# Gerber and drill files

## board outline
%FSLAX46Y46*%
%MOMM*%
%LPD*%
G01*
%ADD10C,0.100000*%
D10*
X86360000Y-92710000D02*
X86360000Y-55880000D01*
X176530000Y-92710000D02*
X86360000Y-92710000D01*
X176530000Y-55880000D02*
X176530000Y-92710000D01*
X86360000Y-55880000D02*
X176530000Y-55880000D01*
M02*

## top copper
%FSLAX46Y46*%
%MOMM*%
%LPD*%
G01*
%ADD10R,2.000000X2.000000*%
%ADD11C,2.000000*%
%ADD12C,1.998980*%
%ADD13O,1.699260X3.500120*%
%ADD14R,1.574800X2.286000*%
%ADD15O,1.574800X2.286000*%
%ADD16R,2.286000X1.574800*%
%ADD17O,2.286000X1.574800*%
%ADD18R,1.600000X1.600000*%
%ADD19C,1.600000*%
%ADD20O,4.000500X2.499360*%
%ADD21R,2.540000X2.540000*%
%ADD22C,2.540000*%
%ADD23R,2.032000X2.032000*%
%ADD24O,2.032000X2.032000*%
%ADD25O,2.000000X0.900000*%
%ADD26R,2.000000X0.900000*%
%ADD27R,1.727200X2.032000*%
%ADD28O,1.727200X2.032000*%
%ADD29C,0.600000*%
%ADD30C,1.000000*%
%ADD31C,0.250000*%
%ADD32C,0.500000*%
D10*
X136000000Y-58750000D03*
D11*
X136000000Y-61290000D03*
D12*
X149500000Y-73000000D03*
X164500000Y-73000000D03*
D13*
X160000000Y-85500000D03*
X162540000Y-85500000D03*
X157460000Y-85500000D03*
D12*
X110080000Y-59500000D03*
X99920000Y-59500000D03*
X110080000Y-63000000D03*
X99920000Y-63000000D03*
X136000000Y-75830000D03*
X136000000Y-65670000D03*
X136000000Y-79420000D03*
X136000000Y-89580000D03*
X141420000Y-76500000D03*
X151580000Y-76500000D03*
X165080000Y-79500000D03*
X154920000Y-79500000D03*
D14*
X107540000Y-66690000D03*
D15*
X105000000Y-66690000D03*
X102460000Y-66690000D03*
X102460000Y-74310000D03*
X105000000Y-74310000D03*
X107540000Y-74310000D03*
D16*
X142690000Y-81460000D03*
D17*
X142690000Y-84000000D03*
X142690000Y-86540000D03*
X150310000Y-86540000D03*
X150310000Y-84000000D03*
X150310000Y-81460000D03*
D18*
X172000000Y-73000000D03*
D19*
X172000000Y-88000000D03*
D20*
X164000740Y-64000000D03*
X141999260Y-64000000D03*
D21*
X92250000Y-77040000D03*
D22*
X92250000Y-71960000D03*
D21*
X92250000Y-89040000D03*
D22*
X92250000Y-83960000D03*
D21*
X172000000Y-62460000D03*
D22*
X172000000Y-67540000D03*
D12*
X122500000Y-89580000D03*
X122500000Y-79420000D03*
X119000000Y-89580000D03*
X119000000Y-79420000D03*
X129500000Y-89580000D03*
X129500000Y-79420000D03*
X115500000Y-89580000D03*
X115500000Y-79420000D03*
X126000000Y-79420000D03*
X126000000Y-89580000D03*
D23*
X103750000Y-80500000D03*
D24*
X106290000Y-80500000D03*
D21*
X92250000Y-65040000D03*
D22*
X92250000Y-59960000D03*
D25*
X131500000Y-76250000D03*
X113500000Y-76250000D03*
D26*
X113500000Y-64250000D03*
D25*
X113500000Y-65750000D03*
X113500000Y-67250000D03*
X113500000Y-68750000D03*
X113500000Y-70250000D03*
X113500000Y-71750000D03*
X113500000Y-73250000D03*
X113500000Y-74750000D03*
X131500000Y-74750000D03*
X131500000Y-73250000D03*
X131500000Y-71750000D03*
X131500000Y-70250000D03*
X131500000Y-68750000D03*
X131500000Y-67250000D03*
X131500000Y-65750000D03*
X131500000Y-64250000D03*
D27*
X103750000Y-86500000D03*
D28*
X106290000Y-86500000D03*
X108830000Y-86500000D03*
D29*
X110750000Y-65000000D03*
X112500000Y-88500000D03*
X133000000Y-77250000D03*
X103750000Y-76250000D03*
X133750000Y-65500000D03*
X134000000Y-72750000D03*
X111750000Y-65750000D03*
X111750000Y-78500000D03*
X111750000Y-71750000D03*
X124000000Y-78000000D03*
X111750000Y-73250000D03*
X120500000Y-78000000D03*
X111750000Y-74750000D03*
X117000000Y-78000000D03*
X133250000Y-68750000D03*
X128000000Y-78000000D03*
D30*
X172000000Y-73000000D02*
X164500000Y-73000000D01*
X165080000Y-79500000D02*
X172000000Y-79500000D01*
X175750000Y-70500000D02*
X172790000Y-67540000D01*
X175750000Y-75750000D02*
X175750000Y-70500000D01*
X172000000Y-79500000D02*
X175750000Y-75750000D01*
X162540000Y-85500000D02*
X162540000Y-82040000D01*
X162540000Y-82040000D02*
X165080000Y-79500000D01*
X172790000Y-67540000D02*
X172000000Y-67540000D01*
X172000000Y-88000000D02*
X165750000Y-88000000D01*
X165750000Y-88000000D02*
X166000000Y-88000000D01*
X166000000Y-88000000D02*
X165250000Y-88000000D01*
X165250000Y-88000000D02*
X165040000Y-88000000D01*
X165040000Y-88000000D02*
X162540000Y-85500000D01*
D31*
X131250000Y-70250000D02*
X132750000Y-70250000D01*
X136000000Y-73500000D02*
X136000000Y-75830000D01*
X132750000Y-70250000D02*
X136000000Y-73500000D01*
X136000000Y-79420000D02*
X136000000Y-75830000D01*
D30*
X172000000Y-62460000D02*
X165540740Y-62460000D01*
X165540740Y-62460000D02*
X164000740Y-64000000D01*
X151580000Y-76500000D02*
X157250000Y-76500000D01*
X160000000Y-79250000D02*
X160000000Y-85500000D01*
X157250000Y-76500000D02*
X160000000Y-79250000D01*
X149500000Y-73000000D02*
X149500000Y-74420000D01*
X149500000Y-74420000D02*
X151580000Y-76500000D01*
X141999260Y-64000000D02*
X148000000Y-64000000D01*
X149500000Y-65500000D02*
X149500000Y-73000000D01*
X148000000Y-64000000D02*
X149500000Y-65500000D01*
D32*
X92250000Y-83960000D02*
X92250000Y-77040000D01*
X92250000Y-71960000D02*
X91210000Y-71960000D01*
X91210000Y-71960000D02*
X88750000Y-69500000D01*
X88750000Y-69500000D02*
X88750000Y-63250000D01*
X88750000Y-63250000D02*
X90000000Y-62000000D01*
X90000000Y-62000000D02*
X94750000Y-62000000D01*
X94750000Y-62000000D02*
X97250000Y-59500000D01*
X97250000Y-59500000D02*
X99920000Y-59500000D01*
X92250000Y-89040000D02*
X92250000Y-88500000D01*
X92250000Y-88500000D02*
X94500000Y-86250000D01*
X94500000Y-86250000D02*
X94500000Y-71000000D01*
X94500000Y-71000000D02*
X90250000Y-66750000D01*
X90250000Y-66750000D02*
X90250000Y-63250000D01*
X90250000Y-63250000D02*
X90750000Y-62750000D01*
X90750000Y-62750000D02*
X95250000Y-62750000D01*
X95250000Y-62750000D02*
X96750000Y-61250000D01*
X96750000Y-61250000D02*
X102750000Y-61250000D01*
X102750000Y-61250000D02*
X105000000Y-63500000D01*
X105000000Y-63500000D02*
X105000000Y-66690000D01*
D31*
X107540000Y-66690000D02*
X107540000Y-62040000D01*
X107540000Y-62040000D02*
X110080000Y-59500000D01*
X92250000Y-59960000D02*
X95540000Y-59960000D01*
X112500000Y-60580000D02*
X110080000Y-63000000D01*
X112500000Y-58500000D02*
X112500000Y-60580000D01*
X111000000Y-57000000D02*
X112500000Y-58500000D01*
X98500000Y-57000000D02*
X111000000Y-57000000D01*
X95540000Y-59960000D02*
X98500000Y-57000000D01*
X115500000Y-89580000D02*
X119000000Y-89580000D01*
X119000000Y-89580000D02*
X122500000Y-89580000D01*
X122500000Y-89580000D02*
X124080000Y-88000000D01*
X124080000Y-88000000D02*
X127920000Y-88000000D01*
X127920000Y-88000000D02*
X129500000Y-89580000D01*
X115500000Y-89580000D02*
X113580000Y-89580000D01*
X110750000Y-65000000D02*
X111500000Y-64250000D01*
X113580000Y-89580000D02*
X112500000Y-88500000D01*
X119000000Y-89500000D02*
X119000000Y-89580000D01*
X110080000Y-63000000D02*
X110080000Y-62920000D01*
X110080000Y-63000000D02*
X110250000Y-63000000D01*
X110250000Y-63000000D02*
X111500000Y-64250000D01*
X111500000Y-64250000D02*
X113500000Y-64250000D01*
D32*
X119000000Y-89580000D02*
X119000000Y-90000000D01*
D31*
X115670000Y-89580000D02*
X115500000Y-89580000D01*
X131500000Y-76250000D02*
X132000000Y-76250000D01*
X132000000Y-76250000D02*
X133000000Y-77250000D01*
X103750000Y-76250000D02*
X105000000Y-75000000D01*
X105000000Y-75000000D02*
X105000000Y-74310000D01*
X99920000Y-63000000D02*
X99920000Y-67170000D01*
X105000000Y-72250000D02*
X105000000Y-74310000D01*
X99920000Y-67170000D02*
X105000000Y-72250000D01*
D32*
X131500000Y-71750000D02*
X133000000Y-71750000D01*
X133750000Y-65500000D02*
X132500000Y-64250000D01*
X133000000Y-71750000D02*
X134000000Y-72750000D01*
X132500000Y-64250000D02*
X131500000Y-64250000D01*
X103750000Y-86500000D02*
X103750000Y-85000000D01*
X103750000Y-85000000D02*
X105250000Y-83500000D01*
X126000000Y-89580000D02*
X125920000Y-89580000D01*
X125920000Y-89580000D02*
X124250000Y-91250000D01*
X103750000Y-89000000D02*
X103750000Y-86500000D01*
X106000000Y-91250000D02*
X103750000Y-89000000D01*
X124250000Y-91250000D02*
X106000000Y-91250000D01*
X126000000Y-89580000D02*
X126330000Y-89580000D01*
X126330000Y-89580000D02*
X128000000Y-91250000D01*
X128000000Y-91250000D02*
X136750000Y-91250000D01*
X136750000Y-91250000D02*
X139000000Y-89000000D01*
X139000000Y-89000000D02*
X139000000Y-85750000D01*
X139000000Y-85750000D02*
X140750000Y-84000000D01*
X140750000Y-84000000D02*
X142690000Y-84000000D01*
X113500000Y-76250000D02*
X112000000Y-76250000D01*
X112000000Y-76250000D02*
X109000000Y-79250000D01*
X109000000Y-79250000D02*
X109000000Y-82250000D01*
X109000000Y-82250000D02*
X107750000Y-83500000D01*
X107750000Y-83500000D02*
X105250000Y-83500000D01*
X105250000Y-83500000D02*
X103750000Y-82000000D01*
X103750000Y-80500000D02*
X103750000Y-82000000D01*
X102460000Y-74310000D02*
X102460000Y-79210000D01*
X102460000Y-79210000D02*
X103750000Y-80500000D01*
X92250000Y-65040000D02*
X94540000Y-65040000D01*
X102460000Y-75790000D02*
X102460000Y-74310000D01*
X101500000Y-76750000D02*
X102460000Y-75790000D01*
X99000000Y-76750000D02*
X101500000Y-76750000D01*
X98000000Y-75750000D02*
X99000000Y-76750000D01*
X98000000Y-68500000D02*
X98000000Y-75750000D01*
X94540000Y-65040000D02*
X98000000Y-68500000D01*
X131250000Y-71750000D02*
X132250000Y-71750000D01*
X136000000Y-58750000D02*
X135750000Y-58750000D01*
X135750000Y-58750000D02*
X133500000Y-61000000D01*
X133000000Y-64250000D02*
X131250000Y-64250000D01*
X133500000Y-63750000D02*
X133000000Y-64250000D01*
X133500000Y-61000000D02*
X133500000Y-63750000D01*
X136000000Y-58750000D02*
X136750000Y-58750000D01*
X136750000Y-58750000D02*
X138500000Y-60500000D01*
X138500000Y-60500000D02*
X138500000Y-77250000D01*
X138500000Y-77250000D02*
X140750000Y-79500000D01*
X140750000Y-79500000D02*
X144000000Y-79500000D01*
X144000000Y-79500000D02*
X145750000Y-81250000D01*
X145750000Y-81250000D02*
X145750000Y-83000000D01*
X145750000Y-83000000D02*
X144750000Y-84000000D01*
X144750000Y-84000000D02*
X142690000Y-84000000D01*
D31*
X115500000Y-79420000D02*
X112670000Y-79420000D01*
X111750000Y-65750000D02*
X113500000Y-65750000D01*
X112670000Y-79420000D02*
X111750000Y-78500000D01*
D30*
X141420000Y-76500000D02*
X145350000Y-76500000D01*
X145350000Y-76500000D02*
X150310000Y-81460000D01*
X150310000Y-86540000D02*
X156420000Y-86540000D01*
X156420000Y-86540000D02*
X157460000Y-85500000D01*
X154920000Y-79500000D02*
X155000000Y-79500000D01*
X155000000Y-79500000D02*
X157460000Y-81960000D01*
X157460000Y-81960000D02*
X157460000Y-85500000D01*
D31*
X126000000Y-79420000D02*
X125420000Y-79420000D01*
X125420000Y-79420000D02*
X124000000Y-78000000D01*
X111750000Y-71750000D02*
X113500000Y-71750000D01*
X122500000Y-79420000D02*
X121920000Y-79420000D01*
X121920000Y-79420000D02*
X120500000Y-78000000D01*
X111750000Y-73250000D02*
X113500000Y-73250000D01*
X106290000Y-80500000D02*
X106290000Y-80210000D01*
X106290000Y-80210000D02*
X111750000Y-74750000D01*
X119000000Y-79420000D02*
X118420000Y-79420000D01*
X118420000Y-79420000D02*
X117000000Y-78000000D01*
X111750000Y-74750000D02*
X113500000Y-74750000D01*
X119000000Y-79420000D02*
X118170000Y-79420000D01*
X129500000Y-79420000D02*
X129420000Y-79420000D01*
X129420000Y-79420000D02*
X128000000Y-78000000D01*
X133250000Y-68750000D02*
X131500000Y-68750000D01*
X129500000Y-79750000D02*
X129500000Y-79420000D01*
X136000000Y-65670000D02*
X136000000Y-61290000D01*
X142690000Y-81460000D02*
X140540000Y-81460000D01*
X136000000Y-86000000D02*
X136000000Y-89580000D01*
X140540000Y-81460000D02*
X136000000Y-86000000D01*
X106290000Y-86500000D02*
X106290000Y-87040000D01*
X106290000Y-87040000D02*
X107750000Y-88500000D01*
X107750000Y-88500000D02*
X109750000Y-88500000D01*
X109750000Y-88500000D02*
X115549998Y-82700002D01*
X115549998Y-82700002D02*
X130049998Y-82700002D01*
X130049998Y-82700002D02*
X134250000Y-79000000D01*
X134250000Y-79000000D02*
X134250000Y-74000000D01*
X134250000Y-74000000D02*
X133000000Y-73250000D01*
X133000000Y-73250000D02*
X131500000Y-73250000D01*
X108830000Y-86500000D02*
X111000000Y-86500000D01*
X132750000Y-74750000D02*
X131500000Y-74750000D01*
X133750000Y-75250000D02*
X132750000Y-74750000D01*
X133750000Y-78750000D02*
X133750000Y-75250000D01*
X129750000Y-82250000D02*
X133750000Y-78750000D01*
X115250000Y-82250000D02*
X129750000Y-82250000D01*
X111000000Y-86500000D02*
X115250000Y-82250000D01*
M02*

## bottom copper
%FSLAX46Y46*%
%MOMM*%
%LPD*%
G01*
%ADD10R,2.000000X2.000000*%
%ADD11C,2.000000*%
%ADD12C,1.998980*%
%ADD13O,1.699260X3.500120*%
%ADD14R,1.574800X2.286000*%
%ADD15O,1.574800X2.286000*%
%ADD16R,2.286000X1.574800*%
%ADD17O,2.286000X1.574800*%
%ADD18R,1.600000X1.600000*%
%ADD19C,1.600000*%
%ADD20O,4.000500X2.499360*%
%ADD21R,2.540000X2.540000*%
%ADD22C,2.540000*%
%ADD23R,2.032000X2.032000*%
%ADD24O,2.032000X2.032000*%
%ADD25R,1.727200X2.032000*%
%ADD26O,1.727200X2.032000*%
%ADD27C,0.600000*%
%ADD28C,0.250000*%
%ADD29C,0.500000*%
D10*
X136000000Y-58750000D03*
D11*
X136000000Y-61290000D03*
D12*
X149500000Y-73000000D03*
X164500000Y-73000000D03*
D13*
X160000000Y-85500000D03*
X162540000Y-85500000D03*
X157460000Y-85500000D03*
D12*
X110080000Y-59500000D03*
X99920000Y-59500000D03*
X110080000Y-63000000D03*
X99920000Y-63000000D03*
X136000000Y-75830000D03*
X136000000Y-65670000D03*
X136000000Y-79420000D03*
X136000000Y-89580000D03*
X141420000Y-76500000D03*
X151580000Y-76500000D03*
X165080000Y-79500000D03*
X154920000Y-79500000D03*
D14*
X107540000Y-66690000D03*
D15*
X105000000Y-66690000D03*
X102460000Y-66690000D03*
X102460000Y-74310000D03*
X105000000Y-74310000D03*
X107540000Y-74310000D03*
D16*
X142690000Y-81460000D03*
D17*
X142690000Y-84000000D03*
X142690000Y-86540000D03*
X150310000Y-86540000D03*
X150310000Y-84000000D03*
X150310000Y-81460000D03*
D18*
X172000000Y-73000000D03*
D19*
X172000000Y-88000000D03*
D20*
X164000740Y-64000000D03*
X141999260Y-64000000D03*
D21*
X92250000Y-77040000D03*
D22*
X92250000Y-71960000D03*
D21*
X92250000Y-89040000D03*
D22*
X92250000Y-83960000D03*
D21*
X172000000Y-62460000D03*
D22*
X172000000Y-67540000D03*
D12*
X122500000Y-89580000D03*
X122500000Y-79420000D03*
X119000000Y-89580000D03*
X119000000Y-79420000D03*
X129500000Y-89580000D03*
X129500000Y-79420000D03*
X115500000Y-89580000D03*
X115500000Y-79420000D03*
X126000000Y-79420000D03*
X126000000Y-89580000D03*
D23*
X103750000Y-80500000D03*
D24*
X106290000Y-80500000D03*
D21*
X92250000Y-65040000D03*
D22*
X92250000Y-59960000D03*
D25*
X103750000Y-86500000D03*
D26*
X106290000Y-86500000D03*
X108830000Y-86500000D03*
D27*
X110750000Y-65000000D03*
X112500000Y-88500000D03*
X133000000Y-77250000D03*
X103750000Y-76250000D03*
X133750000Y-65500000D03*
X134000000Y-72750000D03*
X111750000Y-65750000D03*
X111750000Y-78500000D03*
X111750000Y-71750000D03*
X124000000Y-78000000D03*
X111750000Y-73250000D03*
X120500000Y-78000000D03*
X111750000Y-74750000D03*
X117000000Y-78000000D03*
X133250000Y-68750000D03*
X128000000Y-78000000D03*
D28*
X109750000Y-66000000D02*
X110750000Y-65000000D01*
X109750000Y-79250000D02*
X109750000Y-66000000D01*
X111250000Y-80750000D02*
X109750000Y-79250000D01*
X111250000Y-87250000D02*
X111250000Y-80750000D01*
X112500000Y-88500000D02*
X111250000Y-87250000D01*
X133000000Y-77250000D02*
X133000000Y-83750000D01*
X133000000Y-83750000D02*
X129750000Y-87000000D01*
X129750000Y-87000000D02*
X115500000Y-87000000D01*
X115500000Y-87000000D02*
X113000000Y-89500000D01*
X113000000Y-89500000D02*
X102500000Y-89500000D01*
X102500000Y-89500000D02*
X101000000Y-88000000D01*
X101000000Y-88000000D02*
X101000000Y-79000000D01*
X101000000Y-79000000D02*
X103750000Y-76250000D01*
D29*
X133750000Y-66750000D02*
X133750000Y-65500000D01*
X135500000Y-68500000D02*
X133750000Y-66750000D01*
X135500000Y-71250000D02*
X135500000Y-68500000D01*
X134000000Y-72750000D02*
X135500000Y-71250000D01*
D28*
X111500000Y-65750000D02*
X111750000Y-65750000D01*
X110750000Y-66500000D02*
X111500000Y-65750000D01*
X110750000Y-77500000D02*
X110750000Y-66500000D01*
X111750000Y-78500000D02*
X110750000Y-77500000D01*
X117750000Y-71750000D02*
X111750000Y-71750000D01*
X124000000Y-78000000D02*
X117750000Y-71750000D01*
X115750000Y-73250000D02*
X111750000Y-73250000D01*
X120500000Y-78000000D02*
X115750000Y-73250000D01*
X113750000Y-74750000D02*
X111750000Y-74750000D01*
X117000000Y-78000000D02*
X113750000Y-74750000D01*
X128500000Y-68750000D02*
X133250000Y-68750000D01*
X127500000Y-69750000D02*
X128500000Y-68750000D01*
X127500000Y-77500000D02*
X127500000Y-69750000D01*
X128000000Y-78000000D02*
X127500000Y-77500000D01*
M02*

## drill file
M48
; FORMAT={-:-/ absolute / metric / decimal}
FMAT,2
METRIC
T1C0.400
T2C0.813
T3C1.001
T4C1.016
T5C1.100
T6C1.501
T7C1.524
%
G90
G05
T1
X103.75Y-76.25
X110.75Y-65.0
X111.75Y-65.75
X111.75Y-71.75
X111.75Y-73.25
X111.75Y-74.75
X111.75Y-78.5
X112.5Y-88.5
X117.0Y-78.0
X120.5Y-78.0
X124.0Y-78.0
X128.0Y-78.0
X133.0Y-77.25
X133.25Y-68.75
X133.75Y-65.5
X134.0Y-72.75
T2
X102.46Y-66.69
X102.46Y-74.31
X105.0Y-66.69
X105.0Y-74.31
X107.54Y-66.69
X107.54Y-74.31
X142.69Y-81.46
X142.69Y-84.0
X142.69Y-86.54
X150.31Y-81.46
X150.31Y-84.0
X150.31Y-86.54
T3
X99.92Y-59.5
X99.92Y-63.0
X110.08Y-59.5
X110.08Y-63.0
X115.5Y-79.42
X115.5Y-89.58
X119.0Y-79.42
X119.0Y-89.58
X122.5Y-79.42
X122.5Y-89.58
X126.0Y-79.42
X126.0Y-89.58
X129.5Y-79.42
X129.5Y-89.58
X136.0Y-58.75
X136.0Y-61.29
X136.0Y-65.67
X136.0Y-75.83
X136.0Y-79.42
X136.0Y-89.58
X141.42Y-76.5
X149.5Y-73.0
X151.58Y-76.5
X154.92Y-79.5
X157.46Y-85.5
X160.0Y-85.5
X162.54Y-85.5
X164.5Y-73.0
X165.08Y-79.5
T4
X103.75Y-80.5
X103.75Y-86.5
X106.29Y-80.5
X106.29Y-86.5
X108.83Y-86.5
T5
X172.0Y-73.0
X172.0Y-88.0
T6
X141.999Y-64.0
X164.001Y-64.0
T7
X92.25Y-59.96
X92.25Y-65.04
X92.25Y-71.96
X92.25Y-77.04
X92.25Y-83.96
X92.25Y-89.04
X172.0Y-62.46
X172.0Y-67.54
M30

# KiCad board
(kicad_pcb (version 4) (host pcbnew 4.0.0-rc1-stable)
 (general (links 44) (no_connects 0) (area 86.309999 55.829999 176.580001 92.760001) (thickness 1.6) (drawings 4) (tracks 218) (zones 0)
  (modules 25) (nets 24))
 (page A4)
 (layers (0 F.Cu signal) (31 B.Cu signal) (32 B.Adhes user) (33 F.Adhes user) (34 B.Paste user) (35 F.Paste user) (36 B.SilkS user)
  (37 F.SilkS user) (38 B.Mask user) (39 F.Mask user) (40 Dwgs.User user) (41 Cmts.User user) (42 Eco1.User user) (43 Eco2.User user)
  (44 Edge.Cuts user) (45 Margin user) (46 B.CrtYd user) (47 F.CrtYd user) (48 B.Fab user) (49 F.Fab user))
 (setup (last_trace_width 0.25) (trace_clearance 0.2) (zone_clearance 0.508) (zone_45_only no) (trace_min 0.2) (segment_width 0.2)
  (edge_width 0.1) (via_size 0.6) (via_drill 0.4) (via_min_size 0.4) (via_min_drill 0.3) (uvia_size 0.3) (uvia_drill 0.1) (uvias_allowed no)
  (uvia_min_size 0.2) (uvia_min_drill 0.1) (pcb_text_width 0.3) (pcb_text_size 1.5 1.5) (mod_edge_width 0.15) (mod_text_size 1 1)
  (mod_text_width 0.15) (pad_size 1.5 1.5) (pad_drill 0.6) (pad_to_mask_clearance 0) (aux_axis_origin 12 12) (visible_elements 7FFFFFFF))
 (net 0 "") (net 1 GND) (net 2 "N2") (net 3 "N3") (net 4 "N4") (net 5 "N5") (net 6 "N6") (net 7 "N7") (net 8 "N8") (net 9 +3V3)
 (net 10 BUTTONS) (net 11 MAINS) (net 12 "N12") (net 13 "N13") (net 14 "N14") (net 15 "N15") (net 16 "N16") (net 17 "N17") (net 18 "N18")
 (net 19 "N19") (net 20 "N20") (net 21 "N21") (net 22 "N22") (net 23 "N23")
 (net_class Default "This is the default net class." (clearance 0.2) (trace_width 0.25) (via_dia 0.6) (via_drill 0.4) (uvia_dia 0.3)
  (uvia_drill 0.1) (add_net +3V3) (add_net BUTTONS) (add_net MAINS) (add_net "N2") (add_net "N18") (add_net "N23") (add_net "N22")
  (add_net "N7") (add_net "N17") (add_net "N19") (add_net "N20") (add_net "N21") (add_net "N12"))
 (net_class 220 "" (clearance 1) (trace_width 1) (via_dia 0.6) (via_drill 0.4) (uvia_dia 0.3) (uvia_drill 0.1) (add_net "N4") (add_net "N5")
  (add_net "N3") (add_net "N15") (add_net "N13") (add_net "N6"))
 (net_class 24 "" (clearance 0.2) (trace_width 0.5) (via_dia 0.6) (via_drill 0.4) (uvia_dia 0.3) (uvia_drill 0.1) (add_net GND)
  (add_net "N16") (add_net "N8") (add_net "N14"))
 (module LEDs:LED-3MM (layer F.Cu) (at 136 58.75 270)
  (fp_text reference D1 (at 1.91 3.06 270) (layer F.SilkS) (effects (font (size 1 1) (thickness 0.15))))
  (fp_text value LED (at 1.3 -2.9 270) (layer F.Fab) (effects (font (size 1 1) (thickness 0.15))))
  (pad 1 thru_hole rect (at 0 0) (size 2 2) (drill 1.00076) (layers *.Cu *.Mask F.SilkS) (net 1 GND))
  (pad 2 thru_hole circle (at 2.54 0 270) (size 2 2) (drill 1.00076) (layers *.Cu *.Mask F.SilkS) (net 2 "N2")))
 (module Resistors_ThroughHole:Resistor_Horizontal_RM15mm (layer F.Cu) (at 157 73)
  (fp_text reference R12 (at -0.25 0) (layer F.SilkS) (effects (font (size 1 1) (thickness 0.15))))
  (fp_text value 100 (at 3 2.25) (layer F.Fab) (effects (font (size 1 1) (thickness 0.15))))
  (pad 1 thru_hole circle (at -7.5 0) (size 1.99898 1.99898) (drill 1.00076) (layers *.Cu *.SilkS *.Mask) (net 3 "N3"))
  (pad 2 thru_hole circle (at 7.5 0) (size 1.99898 1.99898) (drill 1.00076) (layers *.Cu *.SilkS *.Mask) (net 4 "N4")))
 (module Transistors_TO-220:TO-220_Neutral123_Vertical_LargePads (layer F.Cu) (at 160 85.5 180)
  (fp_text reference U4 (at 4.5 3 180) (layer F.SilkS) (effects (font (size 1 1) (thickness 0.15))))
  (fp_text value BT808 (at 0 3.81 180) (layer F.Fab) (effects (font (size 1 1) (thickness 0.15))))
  (pad 2 thru_hole oval (at 0 0 270) (size 3.50012 1.69926) (drill 1.00076) (layers *.Cu *.Mask F.SilkS) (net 3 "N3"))
  (pad 1 thru_hole oval (at -2.54 0 270) (size 3.50012 1.69926) (drill 1.00076) (layers *.Cu *.Mask F.SilkS) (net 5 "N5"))
  (pad 3 thru_hole oval (at 2.54 0 270) (size 3.50012 1.69926) (drill 1.00076) (layers *.Cu *.Mask F.SilkS) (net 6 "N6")))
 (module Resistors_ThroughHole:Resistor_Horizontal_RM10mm (layer F.Cu) (at 105 59.5 180)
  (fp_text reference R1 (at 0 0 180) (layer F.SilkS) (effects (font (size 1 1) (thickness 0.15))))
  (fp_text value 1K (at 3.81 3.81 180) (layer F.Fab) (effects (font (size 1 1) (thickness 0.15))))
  (pad 1 thru_hole circle (at -5.08 0 180) (size 1.99898 1.99898) (drill 1.00076) (layers *.Cu *.SilkS *.Mask) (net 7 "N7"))
  (pad 2 thru_hole circle (at 5.08 0 180) (size 1.99898 1.99898) (drill 1.00076) (layers *.Cu *.SilkS *.Mask) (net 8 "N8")))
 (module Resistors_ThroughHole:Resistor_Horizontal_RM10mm (layer F.Cu) (at 105 63 180)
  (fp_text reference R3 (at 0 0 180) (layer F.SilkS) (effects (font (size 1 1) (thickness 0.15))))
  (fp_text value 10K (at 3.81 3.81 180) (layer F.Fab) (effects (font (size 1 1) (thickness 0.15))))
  (pad 1 thru_hole circle (at -5.08 0 180) (size 1.99898 1.99898) (drill 1.00076) (layers *.Cu *.SilkS *.Mask) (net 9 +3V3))
  (pad 2 thru_hole circle (at 5.08 0 180) (size 1.99898 1.99898) (drill 1.00076) (layers *.Cu *.SilkS *.Mask) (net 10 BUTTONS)))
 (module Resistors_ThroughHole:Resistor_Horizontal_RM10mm (layer F.Cu) (at 136 70.75 90)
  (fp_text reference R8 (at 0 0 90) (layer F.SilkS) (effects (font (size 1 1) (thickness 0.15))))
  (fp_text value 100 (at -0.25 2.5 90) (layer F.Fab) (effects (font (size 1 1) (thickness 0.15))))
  (pad 1 thru_hole circle (at -5.08 0 90) (size 1.99898 1.99898) (drill 1.00076) (layers *.Cu *.SilkS *.Mask) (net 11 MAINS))
  (pad 2 thru_hole circle (at 5.08 0 90) (size 1.99898 1.99898) (drill 1.00076) (layers *.Cu *.SilkS *.Mask) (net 2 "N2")))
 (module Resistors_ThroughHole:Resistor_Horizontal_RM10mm (layer F.Cu) (at 136 84.5 270)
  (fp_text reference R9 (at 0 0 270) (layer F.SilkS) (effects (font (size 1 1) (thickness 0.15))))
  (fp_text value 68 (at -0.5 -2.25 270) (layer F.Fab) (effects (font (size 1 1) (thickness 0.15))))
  (pad 1 thru_hole circle (at -5.08 0 270) (size 1.99898 1.99898) (drill 1.00076) (layers *.Cu *.SilkS *.Mask) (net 11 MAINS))
  (pad 2 thru_hole circle (at 5.08 0 270) (size 1.99898 1.99898) (drill 1.00076) (layers *.Cu *.SilkS *.Mask) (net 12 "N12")))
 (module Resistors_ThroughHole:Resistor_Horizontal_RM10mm (layer F.Cu) (at 146.5 76.5)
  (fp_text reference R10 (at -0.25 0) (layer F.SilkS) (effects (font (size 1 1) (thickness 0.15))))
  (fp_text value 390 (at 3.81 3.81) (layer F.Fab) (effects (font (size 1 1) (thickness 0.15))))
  (pad 1 thru_hole circle (at -5.08 0) (size 1.99898 1.99898) (drill 1.00076) (layers *.Cu *.SilkS *.Mask) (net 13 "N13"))
  (pad 2 thru_hole circle (at 5.08 0) (size 1.99898 1.99898) (drill 1.00076) (layers *.Cu *.SilkS *.Mask) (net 3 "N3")))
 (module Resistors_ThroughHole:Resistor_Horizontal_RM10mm (layer F.Cu) (at 160 79.5 180)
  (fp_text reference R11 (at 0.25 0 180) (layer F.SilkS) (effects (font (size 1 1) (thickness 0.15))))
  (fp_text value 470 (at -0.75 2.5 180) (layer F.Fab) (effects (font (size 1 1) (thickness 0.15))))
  (pad 1 thru_hole circle (at -5.08 0 180) (size 1.99898 1.99898) (drill 1.00076) (layers *.Cu *.SilkS *.Mask) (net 5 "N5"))
  (pad 2 thru_hole circle (at 5.08 0 180) (size 1.99898 1.99898) (drill 1.00076) (layers *.Cu *.SilkS *.Mask) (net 6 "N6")))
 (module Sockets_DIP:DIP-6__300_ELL (layer F.Cu) (at 105 70.5 180)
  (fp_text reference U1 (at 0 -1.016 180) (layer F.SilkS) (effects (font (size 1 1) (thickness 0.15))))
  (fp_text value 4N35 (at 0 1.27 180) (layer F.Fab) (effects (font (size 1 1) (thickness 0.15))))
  (pad 1 thru_hole rect (at -2.54 3.81 180) (size 1.5748 2.286) (drill 0.8128) (layers *.Cu *.Mask F.SilkS) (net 7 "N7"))
  (pad 2 thru_hole oval (at 0 3.81 180) (size 1.5748 2.286) (drill 0.8128) (layers *.Cu *.Mask F.SilkS) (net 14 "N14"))
  (pad 3 thru_hole oval (at 2.54 3.81 180) (size 1.5748 2.286) (drill 0.8128) (layers *.Cu *.Mask F.SilkS))
  (pad 4 thru_hole oval (at 2.54 -3.81 180) (size 1.5748 2.286) (drill 0.8128) (layers *.Cu *.Mask F.SilkS) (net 1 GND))
  (pad 5 thru_hole oval (at 0 -3.81 180) (size 1.5748 2.286) (drill 0.8128) (layers *.Cu *.Mask F.SilkS) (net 10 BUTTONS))
  (pad 6 thru_hole oval (at -2.54 -3.81 180) (size 1.5748 2.286) (drill 0.8128) (layers *.Cu *.Mask F.SilkS)))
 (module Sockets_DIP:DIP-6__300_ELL (layer F.Cu) (at 146.5 84 270)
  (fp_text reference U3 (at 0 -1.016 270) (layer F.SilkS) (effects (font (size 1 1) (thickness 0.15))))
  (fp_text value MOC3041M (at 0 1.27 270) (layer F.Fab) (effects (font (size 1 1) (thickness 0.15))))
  (pad 1 thru_hole rect (at -2.54 3.81 270) (size 1.5748 2.286) (drill 0.8128) (layers *.Cu *.Mask F.SilkS) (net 12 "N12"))
  (pad 2 thru_hole oval (at 0 3.81 270) (size 1.5748 2.286) (drill 0.8128) (layers *.Cu *.Mask F.SilkS) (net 1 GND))
  (pad 3 thru_hole oval (at 2.54 3.81 270) (size 1.5748 2.286) (drill 0.8128) (layers *.Cu *.Mask F.SilkS))
  (pad 4 thru_hole oval (at 2.54 -3.81 270) (size 1.5748 2.286) (drill 0.8128) (layers *.Cu *.Mask F.SilkS) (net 6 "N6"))
  (pad 5 thru_hole oval (at 0 -3.81 270) (size 1.5748 2.286) (drill 0.8128) (layers *.Cu *.Mask F.SilkS))
  (pad 6 thru_hole oval (at -2.54 -3.81 270) (size 1.5748 2.286) (drill 0.8128) (layers *.Cu *.Mask F.SilkS) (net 13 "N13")))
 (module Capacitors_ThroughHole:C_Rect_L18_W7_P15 (layer F.Cu) (at 172 73 270)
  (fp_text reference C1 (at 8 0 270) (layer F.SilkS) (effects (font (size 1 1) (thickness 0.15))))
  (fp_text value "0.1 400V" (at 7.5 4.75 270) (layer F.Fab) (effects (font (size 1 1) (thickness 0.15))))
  (pad 1 thru_hole rect (at 0 0 270) (size 1.6 1.6) (drill 1.1) (layers *.Cu *.Mask F.SilkS) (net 4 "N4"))
  (pad 2 thru_hole circle (at 15 0 270) (size 1.6 1.6) (drill 1.1) (layers *.Cu *.Mask F.SilkS) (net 5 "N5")))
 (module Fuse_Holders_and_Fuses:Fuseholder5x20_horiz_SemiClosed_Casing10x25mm (layer F.Cu) (at 153 64)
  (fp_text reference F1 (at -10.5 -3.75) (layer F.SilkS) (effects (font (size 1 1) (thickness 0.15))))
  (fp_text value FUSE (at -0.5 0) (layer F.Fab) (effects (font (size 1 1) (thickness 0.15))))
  (pad 2 thru_hole oval (at 11.00074 0 270) (size 2.49936 4.0005) (drill 1.50114) (layers *.Cu *.Mask F.SilkS) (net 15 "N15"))
  (pad 1 thru_hole oval (at -11.00074 0 270) (size 2.49936 4.0005) (drill 1.50114) (layers *.Cu *.Mask F.SilkS) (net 3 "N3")))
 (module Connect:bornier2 (layer F.Cu) (at 92.25 74.5 90)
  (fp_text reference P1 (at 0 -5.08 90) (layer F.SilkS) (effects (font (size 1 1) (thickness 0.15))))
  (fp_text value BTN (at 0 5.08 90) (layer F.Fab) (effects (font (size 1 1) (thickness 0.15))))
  (pad 1 thru_hole rect (at -2.54 0 90) (size 2.54 2.54) (drill 1.524) (layers *.Cu *.Mask F.SilkS) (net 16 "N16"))
  (pad 2 thru_hole circle (at 2.54 0 90) (size 2.54 2.54) (drill 1.524) (layers *.Cu *.Mask F.SilkS) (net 8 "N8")))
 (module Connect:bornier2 (layer F.Cu) (at 92.25 86.5 90)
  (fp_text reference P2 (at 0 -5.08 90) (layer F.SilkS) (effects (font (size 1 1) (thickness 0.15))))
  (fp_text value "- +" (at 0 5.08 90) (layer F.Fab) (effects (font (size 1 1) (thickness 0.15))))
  (pad 1 thru_hole rect (at -2.54 0 90) (size 2.54 2.54) (drill 1.524) (layers *.Cu *.Mask F.SilkS) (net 14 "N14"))
  (pad 2 thru_hole circle (at 2.54 0 90) (size 2.54 2.54) (drill 1.524) (layers *.Cu *.Mask F.SilkS) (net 16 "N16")))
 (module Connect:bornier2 (layer F.Cu) (at 172 65 270)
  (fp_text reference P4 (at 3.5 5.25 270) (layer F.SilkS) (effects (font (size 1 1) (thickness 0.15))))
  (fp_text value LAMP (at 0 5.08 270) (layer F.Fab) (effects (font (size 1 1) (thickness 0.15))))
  (pad 1 thru_hole rect (at -2.54 0 270) (size 2.54 2.54) (drill 1.524) (layers *.Cu *.Mask F.SilkS) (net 15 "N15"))
  (pad 2 thru_hole circle (at 2.54 0 270) (size 2.54 2.54) (drill 1.524) (layers *.Cu *.Mask F.SilkS) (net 5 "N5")))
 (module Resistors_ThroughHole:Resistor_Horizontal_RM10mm (layer F.Cu) (at 122.5 84.5 90)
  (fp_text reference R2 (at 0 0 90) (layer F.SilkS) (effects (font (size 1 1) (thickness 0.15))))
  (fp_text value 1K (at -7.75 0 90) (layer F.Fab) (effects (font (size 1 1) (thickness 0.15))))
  (pad 1 thru_hole circle (at -5.08 0 90) (size 1.99898 1.99898) (drill 1.00076) (layers *.Cu *.SilkS *.Mask) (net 9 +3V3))
  (pad 2 thru_hole circle (at 5.08 0 90) (size 1.99898 1.99898) (drill 1.00076) (layers *.Cu *.SilkS *.Mask) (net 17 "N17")))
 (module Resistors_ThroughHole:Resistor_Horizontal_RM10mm (layer F.Cu) (at 119 84.5 90)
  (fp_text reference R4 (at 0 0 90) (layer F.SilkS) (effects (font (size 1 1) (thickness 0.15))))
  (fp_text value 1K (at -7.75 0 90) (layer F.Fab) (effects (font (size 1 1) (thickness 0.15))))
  (pad 1 thru_hole circle (at -5.08 0 90) (size 1.99898 1.99898) (drill 1.00076) (layers *.Cu *.SilkS *.Mask) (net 9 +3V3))
  (pad 2 thru_hole circle (at 5.08 0 90) (size 1.99898 1.99898) (drill 1.00076) (layers *.Cu *.SilkS *.Mask) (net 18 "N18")))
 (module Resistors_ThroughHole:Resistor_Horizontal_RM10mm (layer F.Cu) (at 129.5 84.5 90)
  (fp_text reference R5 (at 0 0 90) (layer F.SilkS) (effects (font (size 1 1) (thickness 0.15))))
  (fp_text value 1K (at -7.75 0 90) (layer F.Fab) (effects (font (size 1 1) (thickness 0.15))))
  (pad 1 thru_hole circle (at -5.08 0 90) (size 1.99898 1.99898) (drill 1.00076) (layers *.Cu *.SilkS *.Mask) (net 9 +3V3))
  (pad 2 thru_hole circle (at 5.08 0 90) (size 1.99898 1.99898) (drill 1.00076) (layers *.Cu *.SilkS *.Mask) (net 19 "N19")))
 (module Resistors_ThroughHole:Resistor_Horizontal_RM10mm (layer F.Cu) (at 115.5 84.5 90)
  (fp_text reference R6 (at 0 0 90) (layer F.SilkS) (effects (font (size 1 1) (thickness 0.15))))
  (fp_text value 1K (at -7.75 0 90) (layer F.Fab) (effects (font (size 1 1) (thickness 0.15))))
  (pad 1 thru_hole circle (at -5.08 0 90) (size 1.99898 1.99898) (drill 1.00076) (layers *.Cu *.SilkS *.Mask) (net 9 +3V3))
  (pad 2 thru_hole circle (at 5.08 0 90) (size 1.99898 1.99898) (drill 1.00076) (layers *.Cu *.SilkS *.Mask) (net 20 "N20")))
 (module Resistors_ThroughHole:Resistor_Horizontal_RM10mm (layer F.Cu) (at 126 84.5 270)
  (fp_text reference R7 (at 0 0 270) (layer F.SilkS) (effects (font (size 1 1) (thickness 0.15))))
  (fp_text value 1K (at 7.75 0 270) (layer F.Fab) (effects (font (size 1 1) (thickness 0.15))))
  (pad 1 thru_hole circle (at -5.08 0 270) (size 1.99898 1.99898) (drill 1.00076) (layers *.Cu *.SilkS *.Mask) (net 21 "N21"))
  (pad 2 thru_hole circle (at 5.08 0 270) (size 1.99898 1.99898) (drill 1.00076) (layers *.Cu *.SilkS *.Mask) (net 1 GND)))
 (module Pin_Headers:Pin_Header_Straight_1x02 (layer F.Cu) (at 103.75 80.5 90)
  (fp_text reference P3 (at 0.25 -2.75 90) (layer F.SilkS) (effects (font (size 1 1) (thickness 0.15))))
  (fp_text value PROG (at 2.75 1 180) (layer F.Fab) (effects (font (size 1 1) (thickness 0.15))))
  (pad 1 thru_hole rect (at 0 0 90) (size 2.032 2.032) (drill 1.016) (layers *.Cu *.Mask F.SilkS) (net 1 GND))
  (pad 2 thru_hole oval (at 0 2.54 90) (size 2.032 2.032) (drill 1.016) (layers *.Cu *.Mask F.SilkS) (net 18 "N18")))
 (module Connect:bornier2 (layer F.Cu) (at 92.25 62.5 90)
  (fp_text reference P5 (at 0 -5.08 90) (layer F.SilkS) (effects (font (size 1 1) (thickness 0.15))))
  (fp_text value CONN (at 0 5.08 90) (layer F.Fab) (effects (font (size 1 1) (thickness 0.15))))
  (pad 1 thru_hole rect (at -2.54 0 90) (size 2.54 2.54) (drill 1.524) (layers *.Cu *.Mask F.SilkS) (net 1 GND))
  (pad 2 thru_hole circle (at 2.54 0 90) (size 2.54 2.54) (drill 1.524) (layers *.Cu *.Mask F.SilkS) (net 9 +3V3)))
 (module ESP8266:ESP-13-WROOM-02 (layer F.Cu) (at 113.5 64.25)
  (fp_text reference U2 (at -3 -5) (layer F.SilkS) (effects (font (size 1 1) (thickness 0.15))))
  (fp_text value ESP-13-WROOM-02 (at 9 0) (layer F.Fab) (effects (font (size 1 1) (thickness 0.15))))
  (pad 10 smd oval (at 18 12) (size 2 0.9) (layers F.Cu F.Paste F.Mask) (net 10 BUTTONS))
  (pad 9 smd oval (at 0 12) (size 2 0.9) (layers F.Cu F.Paste F.Mask) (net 1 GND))
  (pad 1 smd rect (at 0 0) (size 2 0.9) (layers F.Cu F.Paste F.Mask) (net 9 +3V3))
  (pad 2 smd oval (at 0 1.5) (size 2 0.9) (layers F.Cu F.Paste F.Mask) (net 20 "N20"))
  (pad 3 smd oval (at 0 3) (size 2 0.9) (layers F.Cu F.Paste F.Mask))
  (pad 4 smd oval (at 0 4.5) (size 2 0.9) (layers F.Cu F.Paste F.Mask))
  (pad 5 smd oval (at 0 6) (size 2 0.9) (layers F.Cu F.Paste F.Mask))
  (pad 6 smd oval (at 0 7.5) (size 2 0.9) (layers F.Cu F.Paste F.Mask) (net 21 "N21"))
  (pad 7 smd oval (at 0 9) (size 2 0.9) (layers F.Cu F.Paste F.Mask) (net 17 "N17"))
  (pad 8 smd oval (at 0 10.5) (size 2 0.9) (layers F.Cu F.Paste F.Mask) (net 18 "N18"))
  (pad 11 smd oval (at 18 10.5) (size 2 0.9) (layers F.Cu F.Paste F.Mask) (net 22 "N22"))
  (pad 12 smd oval (at 18 9) (size 2 0.9) (layers F.Cu F.Paste F.Mask) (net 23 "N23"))
  (pad 13 smd oval (at 18 7.5) (size 2 0.9) (layers F.Cu F.Paste F.Mask) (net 1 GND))
  (pad 14 smd oval (at 18 6) (size 2 0.9) (layers F.Cu F.Paste F.Mask) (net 11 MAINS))
  (pad 15 smd oval (at 18 4.5) (size 2 0.9) (layers F.Cu F.Paste F.Mask) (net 19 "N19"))
  (pad 16 smd oval (at 18 3) (size 2 0.9) (layers F.Cu F.Paste F.Mask))
  (pad 17 smd oval (at 18 1.5) (size 2 0.9) (layers F.Cu F.Paste F.Mask))
  (pad 18 smd oval (at 18 0) (size 2 0.9) (layers F.Cu F.Paste F.Mask) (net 1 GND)))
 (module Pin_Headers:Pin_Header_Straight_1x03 (layer F.Cu) (at 103.75 86.5 90)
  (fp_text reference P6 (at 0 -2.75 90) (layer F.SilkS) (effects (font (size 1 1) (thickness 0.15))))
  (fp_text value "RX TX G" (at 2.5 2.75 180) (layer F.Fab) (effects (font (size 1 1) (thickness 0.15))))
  (pad 1 thru_hole rect (at 0 0 90) (size 2.032 1.7272) (drill 1.016) (layers *.Cu *.Mask F.SilkS) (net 1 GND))
  (pad 2 thru_hole oval (at 0 2.54 90) (size 2.032 1.7272) (drill 1.016) (layers *.Cu *.Mask F.SilkS) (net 23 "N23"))
  (pad 3 thru_hole oval (at 0 5.08 90) (size 2.032 1.7272) (drill 1.016) (layers *.Cu *.Mask F.SilkS) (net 22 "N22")))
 (gr_line (start 86.36 92.71) (end 86.36 55.88) (angle 90) (layer Edge.Cuts) (width 0.1))
 (gr_line (start 176.53 92.71) (end 86.36 92.71) (angle 90) (layer Edge.Cuts) (width 0.1))
 (gr_line (start 176.53 55.88) (end 176.53 92.71) (angle 90) (layer Edge.Cuts) (width 0.1))
 (gr_line (start 86.36 55.88) (end 176.53 55.88) (angle 90) (layer Edge.Cuts) (width 0.1))
 (segment (start 172 73) (end 164.5 73) (width 1) (layer F.Cu) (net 4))
 (segment (start 165.08 79.5) (end 172 79.5) (width 1) (layer F.Cu) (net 5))
 (segment (start 175.75 70.5) (end 172.79 67.54) (width 1) (layer F.Cu) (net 5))
 (segment (start 175.75 75.75) (end 175.75 70.5) (width 1) (layer F.Cu) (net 5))
 (segment (start 172 79.5) (end 175.75 75.75) (width 1) (layer F.Cu) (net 5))
 (segment (start 162.54 85.5) (end 162.54 82.04) (width 1) (layer F.Cu) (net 5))
 (segment (start 162.54 82.04) (end 165.08 79.5) (width 1) (layer F.Cu) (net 5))
 (segment (start 172.79 67.54) (end 172 67.54) (width 1) (layer F.Cu) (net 5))
 (segment (start 172 88) (end 165.75 88) (width 1) (layer F.Cu) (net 5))
 (segment (start 165.75 88) (end 166 88) (width 1) (layer F.Cu) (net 5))
 (segment (start 166 88) (end 165.25 88) (width 1) (layer F.Cu) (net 5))
 (segment (start 165.25 88) (end 165.04 88) (width 1) (layer F.Cu) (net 5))
 (segment (start 165.04 88) (end 162.54 85.5) (width 1) (layer F.Cu) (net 5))
 (segment (start 131.25 70.25) (end 132.75 70.25) (width 0.25) (layer F.Cu) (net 11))
 (segment (start 136 73.5) (end 136 75.83) (width 0.25) (layer F.Cu) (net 11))
 (segment (start 132.75 70.25) (end 136 73.5) (width 0.25) (layer F.Cu) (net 11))
 (segment (start 136 79.42) (end 136 75.83) (width 0.25) (layer F.Cu) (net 11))
 (segment (start 172 62.46) (end 165.54074 62.46) (width 1) (layer F.Cu) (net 15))
 (segment (start 165.54074 62.46) (end 164.00074 64) (width 1) (layer F.Cu) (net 15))
 (segment (start 151.58 76.5) (end 157.25 76.5) (width 1) (layer F.Cu) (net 3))
 (segment (start 160 79.25) (end 160 85.5) (width 1) (layer F.Cu) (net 3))
 (segment (start 157.25 76.5) (end 160 79.25) (width 1) (layer F.Cu) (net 3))
 (segment (start 149.5 73) (end 149.5 74.42) (width 1) (layer F.Cu) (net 3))
 (segment (start 149.5 74.42) (end 151.58 76.5) (width 1) (layer F.Cu) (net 3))
 (segment (start 141.99926 64) (end 148 64) (width 1) (layer F.Cu) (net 3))
 (segment (start 149.5 65.5) (end 149.5 73) (width 1) (layer F.Cu) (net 3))
 (segment (start 148 64) (end 149.5 65.5) (width 1) (layer F.Cu) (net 3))
 (segment (start 92.25 83.96) (end 92.25 77.04) (width 0.5) (layer F.Cu) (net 16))
 (segment (start 92.25 71.96) (end 91.21 71.96) (width 0.5) (layer F.Cu) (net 8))
 (segment (start 91.21 71.96) (end 88.75 69.5) (width 0.5) (layer F.Cu) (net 8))
 (segment (start 88.75 69.5) (end 88.75 63.25) (width 0.5) (layer F.Cu) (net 8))
 (segment (start 88.75 63.25) (end 90 62) (width 0.5) (layer F.Cu) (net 8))
 (segment (start 90 62) (end 94.75 62) (width 0.5) (layer F.Cu) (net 8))
 (segment (start 94.75 62) (end 97.25 59.5) (width 0.5) (layer F.Cu) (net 8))
 (segment (start 97.25 59.5) (end 99.92 59.5) (width 0.5) (layer F.Cu) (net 8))
 (segment (start 92.25 89.04) (end 92.25 88.5) (width 0.5) (layer F.Cu) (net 14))
 (segment (start 92.25 88.5) (end 94.5 86.25) (width 0.5) (layer F.Cu) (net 14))
 (segment (start 94.5 86.25) (end 94.5 71) (width 0.5) (layer F.Cu) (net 14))
 (segment (start 94.5 71) (end 90.25 66.75) (width 0.5) (layer F.Cu) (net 14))
 (segment (start 90.25 66.75) (end 90.25 63.25) (width 0.5) (layer F.Cu) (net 14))
 (segment (start 90.25 63.25) (end 90.75 62.75) (width 0.5) (layer F.Cu) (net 14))
 (segment (start 90.75 62.75) (end 95.25 62.75) (width 0.5) (layer F.Cu) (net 14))
 (segment (start 95.25 62.75) (end 96.75 61.25) (width 0.5) (layer F.Cu) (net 14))
 (segment (start 96.75 61.25) (end 102.75 61.25) (width 0.5) (layer F.Cu) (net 14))
 (segment (start 102.75 61.25) (end 105 63.5) (width 0.5) (layer F.Cu) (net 14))
 (segment (start 105 63.5) (end 105 66.69) (width 0.5) (layer F.Cu) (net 14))
 (segment (start 107.54 66.69) (end 107.54 62.04) (width 0.25) (layer F.Cu) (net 7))
 (segment (start 107.54 62.04) (end 110.08 59.5) (width 0.25) (layer F.Cu) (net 7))
 (segment (start 92.25 59.96) (end 95.54 59.96) (width 0.25) (layer F.Cu) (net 9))
 (segment (start 112.5 60.58) (end 110.08 63) (width 0.25) (layer F.Cu) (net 9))
 (segment (start 112.5 58.5) (end 112.5 60.58) (width 0.25) (layer F.Cu) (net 9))
 (segment (start 111 57) (end 112.5 58.5) (width 0.25) (layer F.Cu) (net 9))
 (segment (start 98.5 57) (end 111 57) (width 0.25) (layer F.Cu) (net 9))
 (segment (start 95.54 59.96) (end 98.5 57) (width 0.25) (layer F.Cu) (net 9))
 (segment (start 115.5 89.58) (end 119 89.58) (width 0.25) (layer F.Cu) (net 9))
 (segment (start 119 89.58) (end 122.5 89.58) (width 0.25) (layer F.Cu) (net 9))
 (segment (start 122.5 89.58) (end 124.08 88) (width 0.25) (layer F.Cu) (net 9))
 (segment (start 124.08 88) (end 127.92 88) (width 0.25) (layer F.Cu) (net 9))
 (segment (start 127.92 88) (end 129.5 89.58) (width 0.25) (layer F.Cu) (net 9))
 (segment (start 115.5 89.58) (end 113.58 89.58) (width 0.25) (layer F.Cu) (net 9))
 (segment (start 110.75 65) (end 111.5 64.25) (width 0.25) (layer F.Cu) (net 9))
 (via (at 110.75 65) (size 0.6) (drill 0.4) (layers F.Cu B.Cu) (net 9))
 (segment (start 109.75 66) (end 110.75 65) (width 0.25) (layer B.Cu) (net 9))
 (segment (start 109.75 79.25) (end 109.75 66) (width 0.25) (layer B.Cu) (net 9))
 (segment (start 111.25 80.75) (end 109.75 79.25) (width 0.25) (layer B.Cu) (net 9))
 (segment (start 111.25 87.25) (end 111.25 80.75) (width 0.25) (layer B.Cu) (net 9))
 (segment (start 112.5 88.5) (end 111.25 87.25) (width 0.25) (layer B.Cu) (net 9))
 (via (at 112.5 88.5) (size 0.6) (drill 0.4) (layers F.Cu B.Cu) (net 9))
 (segment (start 113.58 89.58) (end 112.5 88.5) (width 0.25) (layer F.Cu) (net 9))
 (segment (start 119 89.5) (end 119 89.58) (width 0.25) (layer F.Cu) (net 9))
 (segment (start 110.08 63) (end 110.08 62.92) (width 0.25) (layer F.Cu) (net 9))
 (segment (start 110.08 63) (end 110.25 63) (width 0.25) (layer F.Cu) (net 9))
 (segment (start 110.25 63) (end 111.5 64.25) (width 0.25) (layer F.Cu) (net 9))
 (segment (start 111.5 64.25) (end 113.5 64.25) (width 0.25) (layer F.Cu) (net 9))
 (segment (start 119 89.58) (end 119 90) (width 0.5) (layer F.Cu) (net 9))
 (segment (start 115.67 89.58) (end 115.5 89.58) (width 0.25) (layer F.Cu) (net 9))
 (segment (start 131.5 76.25) (end 132 76.25) (width 0.25) (layer F.Cu) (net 10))
 (segment (start 132 76.25) (end 133 77.25) (width 0.25) (layer F.Cu) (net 10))
 (via (at 133 77.25) (size 0.6) (drill 0.4) (layers F.Cu B.Cu) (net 10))
 (segment (start 133 77.25) (end 133 83.75) (width 0.25) (layer B.Cu) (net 10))
 (segment (start 133 83.75) (end 129.75 87) (width 0.25) (layer B.Cu) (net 10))
 (segment (start 129.75 87) (end 115.5 87) (width 0.25) (layer B.Cu) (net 10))
 (segment (start 115.5 87) (end 113 89.5) (width 0.25) (layer B.Cu) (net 10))
 (segment (start 113 89.5) (end 102.5 89.5) (width 0.25) (layer B.Cu) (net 10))
 (segment (start 102.5 89.5) (end 101 88) (width 0.25) (layer B.Cu) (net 10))
 (segment (start 101 88) (end 101 79) (width 0.25) (layer B.Cu) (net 10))
 (segment (start 101 79) (end 103.75 76.25) (width 0.25) (layer B.Cu) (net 10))
 (via (at 103.75 76.25) (size 0.6) (drill 0.4) (layers F.Cu B.Cu) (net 10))
 (segment (start 103.75 76.25) (end 105 75) (width 0.25) (layer F.Cu) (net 10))
 (segment (start 105 75) (end 105 74.31) (width 0.25) (layer F.Cu) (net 10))
 (segment (start 99.92 63) (end 99.92 67.17) (width 0.25) (layer F.Cu) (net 10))
 (segment (start 105 72.25) (end 105 74.31) (width 0.25) (layer F.Cu) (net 10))
 (segment (start 99.92 67.17) (end 105 72.25) (width 0.25) (layer F.Cu) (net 10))
 (segment (start 131.5 71.75) (end 133 71.75) (width 0.5) (layer F.Cu) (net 1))
 (segment (start 133.75 65.5) (end 132.5 64.25) (width 0.5) (layer F.Cu) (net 1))
 (via (at 133.75 65.5) (size 0.6) (drill 0.4) (layers F.Cu B.Cu) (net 1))
 (segment (start 133.75 66.75) (end 133.75 65.5) (width 0.5) (layer B.Cu) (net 1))
 (segment (start 135.5 68.5) (end 133.75 66.75) (width 0.5) (layer B.Cu) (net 1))
 (segment (start 135.5 71.25) (end 135.5 68.5) (width 0.5) (layer B.Cu) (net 1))
 (segment (start 134 72.75) (end 135.5 71.25) (width 0.5) (layer B.Cu) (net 1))
 (via (at 134 72.75) (size 0.6) (drill 0.4) (layers F.Cu B.Cu) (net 1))
 (segment (start 133 71.75) (end 134 72.75) (width 0.5) (layer F.Cu) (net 1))
 (segment (start 132.5 64.25) (end 131.5 64.25) (width 0.5) (layer F.Cu) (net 1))
 (segment (start 103.75 86.5) (end 103.75 85) (width 0.5) (layer F.Cu) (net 1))
 (segment (start 103.75 85) (end 105.25 83.5) (width 0.5) (layer F.Cu) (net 1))
 (segment (start 126 89.58) (end 125.92 89.58) (width 0.5) (layer F.Cu) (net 1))
 (segment (start 125.92 89.58) (end 124.25 91.25) (width 0.5) (layer F.Cu) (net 1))
 (segment (start 103.75 89) (end 103.75 86.5) (width 0.5) (layer F.Cu) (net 1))
 (segment (start 106 91.25) (end 103.75 89) (width 0.5) (layer F.Cu) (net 1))
 (segment (start 124.25 91.25) (end 106 91.25) (width 0.5) (layer F.Cu) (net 1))
 (segment (start 126 89.58) (end 126.33 89.58) (width 0.5) (layer F.Cu) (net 1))
 (segment (start 126.33 89.58) (end 128 91.25) (width 0.5) (layer F.Cu) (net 1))
 (segment (start 128 91.25) (end 136.75 91.25) (width 0.5) (layer F.Cu) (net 1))
 (segment (start 136.75 91.25) (end 139 89) (width 0.5) (layer F.Cu) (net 1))
 (segment (start 139 89) (end 139 85.75) (width 0.5) (layer F.Cu) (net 1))
 (segment (start 139 85.75) (end 140.75 84) (width 0.5) (layer F.Cu) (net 1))
 (segment (start 140.75 84) (end 142.69 84) (width 0.5) (layer F.Cu) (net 1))
 (segment (start 113.5 76.25) (end 112 76.25) (width 0.5) (layer F.Cu) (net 1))
 (segment (start 112 76.25) (end 109 79.25) (width 0.5) (layer F.Cu) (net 1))
 (segment (start 109 79.25) (end 109 82.25) (width 0.5) (layer F.Cu) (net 1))
 (segment (start 109 82.25) (end 107.75 83.5) (width 0.5) (layer F.Cu) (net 1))
 (segment (start 107.75 83.5) (end 105.25 83.5) (width 0.5) (layer F.Cu) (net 1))
 (segment (start 105.25 83.5) (end 103.75 82) (width 0.5) (layer F.Cu) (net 1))
 (segment (start 103.75 80.5) (end 103.75 82) (width 0.5) (layer F.Cu) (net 1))
 (segment (start 102.46 74.31) (end 102.46 79.21) (width 0.5) (layer F.Cu) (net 1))
 (segment (start 102.46 79.21) (end 103.75 80.5) (width 0.5) (layer F.Cu) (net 1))
 (segment (start 92.25 65.04) (end 94.54 65.04) (width 0.5) (layer F.Cu) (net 1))
 (segment (start 102.46 75.79) (end 102.46 74.31) (width 0.5) (layer F.Cu) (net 1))
 (segment (start 101.5 76.75) (end 102.46 75.79) (width 0.5) (layer F.Cu) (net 1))
 (segment (start 99 76.75) (end 101.5 76.75) (width 0.5) (layer F.Cu) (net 1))
 (segment (start 98 75.75) (end 99 76.75) (width 0.5) (layer F.Cu) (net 1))
 (segment (start 98 68.5) (end 98 75.75) (width 0.5) (layer F.Cu) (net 1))
 (segment (start 94.54 65.04) (end 98 68.5) (width 0.5) (layer F.Cu) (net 1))
 (segment (start 131.25 71.75) (end 132.25 71.75) (width 0.5) (layer F.Cu) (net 1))
 (segment (start 136 58.75) (end 135.75 58.75) (width 0.5) (layer F.Cu) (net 1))
 (segment (start 135.75 58.75) (end 133.5 61) (width 0.5) (layer F.Cu) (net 1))
 (segment (start 133 64.25) (end 131.25 64.25) (width 0.5) (layer F.Cu) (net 1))
 (segment (start 133.5 63.75) (end 133 64.25) (width 0.5) (layer F.Cu) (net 1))
 (segment (start 133.5 61) (end 133.5 63.75) (width 0.5) (layer F.Cu) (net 1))
 (segment (start 136 58.75) (end 136.75 58.75) (width 0.5) (layer F.Cu) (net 1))
 (segment (start 136.75 58.75) (end 138.5 60.5) (width 0.5) (layer F.Cu) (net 1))
 (segment (start 138.5 60.5) (end 138.5 77.25) (width 0.5) (layer F.Cu) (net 1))
 (segment (start 138.5 77.25) (end 140.75 79.5) (width 0.5) (layer F.Cu) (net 1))
 (segment (start 140.75 79.5) (end 144 79.5) (width 0.5) (layer F.Cu) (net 1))
 (segment (start 144 79.5) (end 145.75 81.25) (width 0.5) (layer F.Cu) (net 1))
 (segment (start 145.75 81.25) (end 145.75 83) (width 0.5) (layer F.Cu) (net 1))
 (segment (start 145.75 83) (end 144.75 84) (width 0.5) (layer F.Cu) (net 1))
 (segment (start 144.75 84) (end 142.69 84) (width 0.5) (layer F.Cu) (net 1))
 (segment (start 115.5 79.42) (end 112.67 79.42) (width 0.25) (layer F.Cu) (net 20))
 (segment (start 111.75 65.75) (end 113.5 65.75) (width 0.25) (layer F.Cu) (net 20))
 (via (at 111.75 65.75) (size 0.6) (drill 0.4) (layers F.Cu B.Cu) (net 20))
 (segment (start 111.5 65.75) (end 111.75 65.75) (width 0.25) (layer B.Cu) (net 20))
 (segment (start 110.75 66.5) (end 111.5 65.75) (width 0.25) (layer B.Cu) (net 20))
 (segment (start 110.75 77.5) (end 110.75 66.5) (width 0.25) (layer B.Cu) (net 20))
 (segment (start 111.75 78.5) (end 110.75 77.5) (width 0.25) (layer B.Cu) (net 20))
 (via (at 111.75 78.5) (size 0.6) (drill 0.4) (layers F.Cu B.Cu) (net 20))
 (segment (start 112.67 79.42) (end 111.75 78.5) (width 0.25) (layer F.Cu) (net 20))
 (segment (start 141.42 76.5) (end 145.35 76.5) (width 1) (layer F.Cu) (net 13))
 (segment (start 145.35 76.5) (end 150.31 81.46) (width 1) (layer F.Cu) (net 13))
 (segment (start 150.31 86.54) (end 156.42 86.54) (width 1) (layer F.Cu) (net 6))
 (segment (start 156.42 86.54) (end 157.46 85.5) (width 1) (layer F.Cu) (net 6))
 (segment (start 154.92 79.5) (end 155 79.5) (width 1) (layer F.Cu) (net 6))
 (segment (start 155 79.5) (end 157.46 81.96) (width 1) (layer F.Cu) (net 6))
 (segment (start 157.46 81.96) (end 157.46 85.5) (width 1) (layer F.Cu) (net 6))
 (segment (start 126 79.42) (end 125.42 79.42) (width 0.25) (layer F.Cu) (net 21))
 (segment (start 125.42 79.42) (end 124 78) (width 0.25) (layer F.Cu) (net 21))
 (segment (start 111.75 71.75) (end 113.5 71.75) (width 0.25) (layer F.Cu) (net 21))
 (via (at 111.75 71.75) (size 0.6) (drill 0.4) (layers F.Cu B.Cu) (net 21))
 (segment (start 117.75 71.75) (end 111.75 71.75) (width 0.25) (layer B.Cu) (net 21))
 (segment (start 124 78) (end 117.75 71.75) (width 0.25) (layer B.Cu) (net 21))
 (via (at 124 78) (size 0.6) (drill 0.4) (layers F.Cu B.Cu) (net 21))
 (segment (start 122.5 79.42) (end 121.92 79.42) (width 0.25) (layer F.Cu) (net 17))
 (segment (start 121.92 79.42) (end 120.5 78) (width 0.25) (layer F.Cu) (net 17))
 (segment (start 111.75 73.25) (end 113.5 73.25) (width 0.25) (layer F.Cu) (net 17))
 (via (at 111.75 73.25) (size 0.6) (drill 0.4) (layers F.Cu B.Cu) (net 17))
 (segment (start 115.75 73.25) (end 111.75 73.25) (width 0.25) (layer B.Cu) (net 17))
 (segment (start 120.5 78) (end 115.75 73.25) (width 0.25) (layer B.Cu) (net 17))
 (via (at 120.5 78) (size 0.6) (drill 0.4) (layers F.Cu B.Cu) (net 17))
 (segment (start 106.29 80.5) (end 106.29 80.21) (width 0.25) (layer F.Cu) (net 18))
 (segment (start 106.29 80.21) (end 111.75 74.75) (width 0.25) (layer F.Cu) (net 18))
 (segment (start 119 79.42) (end 118.42 79.42) (width 0.25) (layer F.Cu) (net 18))
 (segment (start 118.42 79.42) (end 117 78) (width 0.25) (layer F.Cu) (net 18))
 (segment (start 111.75 74.75) (end 113.5 74.75) (width 0.25) (layer F.Cu) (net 18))
 (via (at 111.75 74.75) (size 0.6) (drill 0.4) (layers F.Cu B.Cu) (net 18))
 (segment (start 113.75 74.75) (end 111.75 74.75) (width 0.25) (layer B.Cu) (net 18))
 (segment (start 117 78) (end 113.75 74.75) (width 0.25) (layer B.Cu) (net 18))
 (via (at 117 78) (size 0.6) (drill 0.4) (layers F.Cu B.Cu) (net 18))
 (segment (start 119 79.42) (end 118.17 79.42) (width 0.25) (layer F.Cu) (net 18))
 (segment (start 129.5 79.42) (end 129.42 79.42) (width 0.25) (layer F.Cu) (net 19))
 (segment (start 129.42 79.42) (end 128 78) (width 0.25) (layer F.Cu) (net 19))
 (segment (start 133.25 68.75) (end 131.5 68.75) (width 0.25) (layer F.Cu) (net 19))
 (via (at 133.25 68.75) (size 0.6) (drill 0.4) (layers F.Cu B.Cu) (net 19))
 (segment (start 128.5 68.75) (end 133.25 68.75) (width 0.25) (layer B.Cu) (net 19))
 (segment (start 127.5 69.75) (end 128.5 68.75) (width 0.25) (layer B.Cu) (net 19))
 (segment (start 127.5 77.5) (end 127.5 69.75) (width 0.25) (layer B.Cu) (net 19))
 (segment (start 128 78) (end 127.5 77.5) (width 0.25) (layer B.Cu) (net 19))
 (via (at 128 78) (size 0.6) (drill 0.4) (layers F.Cu B.Cu) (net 19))
 (segment (start 129.5 79.75) (end 129.5 79.42) (width 0.25) (layer F.Cu) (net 19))
 (segment (start 136 65.67) (end 136 61.29) (width 0.25) (layer F.Cu) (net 2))
 (segment (start 142.69 81.46) (end 140.54 81.46) (width 0.25) (layer F.Cu) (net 12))
 (segment (start 136 86) (end 136 89.58) (width 0.25) (layer F.Cu) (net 12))
 (segment (start 140.54 81.46) (end 136 86) (width 0.25) (layer F.Cu) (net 12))
 (segment (start 106.29 86.5) (end 106.29 87.04) (width 0.25) (layer F.Cu) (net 23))
 (segment (start 106.29 87.04) (end 107.75 88.5) (width 0.25) (layer F.Cu) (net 23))
 (segment (start 107.75 88.5) (end 109.75 88.5) (width 0.25) (layer F.Cu) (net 23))
 (segment (start 109.75 88.5) (end 115.549998 82.700002) (width 0.25) (layer F.Cu) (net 23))
 (segment (start 115.549998 82.700002) (end 130.049998 82.700002) (width 0.25) (layer F.Cu) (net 23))
 (segment (start 130.049998 82.700002) (end 134.25 79) (width 0.25) (layer F.Cu) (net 23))
 (segment (start 134.25 79) (end 134.25 74) (width 0.25) (layer F.Cu) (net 23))
 (segment (start 134.25 74) (end 133 73.25) (width 0.25) (layer F.Cu) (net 23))
 (segment (start 133 73.25) (end 131.5 73.25) (width 0.25) (layer F.Cu) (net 23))
 (segment (start 108.83 86.5) (end 111 86.5) (width 0.25) (layer F.Cu) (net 22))
 (segment (start 132.75 74.75) (end 131.5 74.75) (width 0.25) (layer F.Cu) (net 22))
 (segment (start 133.75 75.25) (end 132.75 74.75) (width 0.25) (layer F.Cu) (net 22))
 (segment (start 133.75 78.75) (end 133.75 75.25) (width 0.25) (layer F.Cu) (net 22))
 (segment (start 129.75 82.25) (end 133.75 78.75) (width 0.25) (layer F.Cu) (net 22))
 (segment (start 115.25 82.25) (end 129.75 82.25) (width 0.25) (layer F.Cu) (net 22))
 (segment (start 111 86.5) (end 115.25 82.25) (width 0.25) (layer F.Cu) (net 22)))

